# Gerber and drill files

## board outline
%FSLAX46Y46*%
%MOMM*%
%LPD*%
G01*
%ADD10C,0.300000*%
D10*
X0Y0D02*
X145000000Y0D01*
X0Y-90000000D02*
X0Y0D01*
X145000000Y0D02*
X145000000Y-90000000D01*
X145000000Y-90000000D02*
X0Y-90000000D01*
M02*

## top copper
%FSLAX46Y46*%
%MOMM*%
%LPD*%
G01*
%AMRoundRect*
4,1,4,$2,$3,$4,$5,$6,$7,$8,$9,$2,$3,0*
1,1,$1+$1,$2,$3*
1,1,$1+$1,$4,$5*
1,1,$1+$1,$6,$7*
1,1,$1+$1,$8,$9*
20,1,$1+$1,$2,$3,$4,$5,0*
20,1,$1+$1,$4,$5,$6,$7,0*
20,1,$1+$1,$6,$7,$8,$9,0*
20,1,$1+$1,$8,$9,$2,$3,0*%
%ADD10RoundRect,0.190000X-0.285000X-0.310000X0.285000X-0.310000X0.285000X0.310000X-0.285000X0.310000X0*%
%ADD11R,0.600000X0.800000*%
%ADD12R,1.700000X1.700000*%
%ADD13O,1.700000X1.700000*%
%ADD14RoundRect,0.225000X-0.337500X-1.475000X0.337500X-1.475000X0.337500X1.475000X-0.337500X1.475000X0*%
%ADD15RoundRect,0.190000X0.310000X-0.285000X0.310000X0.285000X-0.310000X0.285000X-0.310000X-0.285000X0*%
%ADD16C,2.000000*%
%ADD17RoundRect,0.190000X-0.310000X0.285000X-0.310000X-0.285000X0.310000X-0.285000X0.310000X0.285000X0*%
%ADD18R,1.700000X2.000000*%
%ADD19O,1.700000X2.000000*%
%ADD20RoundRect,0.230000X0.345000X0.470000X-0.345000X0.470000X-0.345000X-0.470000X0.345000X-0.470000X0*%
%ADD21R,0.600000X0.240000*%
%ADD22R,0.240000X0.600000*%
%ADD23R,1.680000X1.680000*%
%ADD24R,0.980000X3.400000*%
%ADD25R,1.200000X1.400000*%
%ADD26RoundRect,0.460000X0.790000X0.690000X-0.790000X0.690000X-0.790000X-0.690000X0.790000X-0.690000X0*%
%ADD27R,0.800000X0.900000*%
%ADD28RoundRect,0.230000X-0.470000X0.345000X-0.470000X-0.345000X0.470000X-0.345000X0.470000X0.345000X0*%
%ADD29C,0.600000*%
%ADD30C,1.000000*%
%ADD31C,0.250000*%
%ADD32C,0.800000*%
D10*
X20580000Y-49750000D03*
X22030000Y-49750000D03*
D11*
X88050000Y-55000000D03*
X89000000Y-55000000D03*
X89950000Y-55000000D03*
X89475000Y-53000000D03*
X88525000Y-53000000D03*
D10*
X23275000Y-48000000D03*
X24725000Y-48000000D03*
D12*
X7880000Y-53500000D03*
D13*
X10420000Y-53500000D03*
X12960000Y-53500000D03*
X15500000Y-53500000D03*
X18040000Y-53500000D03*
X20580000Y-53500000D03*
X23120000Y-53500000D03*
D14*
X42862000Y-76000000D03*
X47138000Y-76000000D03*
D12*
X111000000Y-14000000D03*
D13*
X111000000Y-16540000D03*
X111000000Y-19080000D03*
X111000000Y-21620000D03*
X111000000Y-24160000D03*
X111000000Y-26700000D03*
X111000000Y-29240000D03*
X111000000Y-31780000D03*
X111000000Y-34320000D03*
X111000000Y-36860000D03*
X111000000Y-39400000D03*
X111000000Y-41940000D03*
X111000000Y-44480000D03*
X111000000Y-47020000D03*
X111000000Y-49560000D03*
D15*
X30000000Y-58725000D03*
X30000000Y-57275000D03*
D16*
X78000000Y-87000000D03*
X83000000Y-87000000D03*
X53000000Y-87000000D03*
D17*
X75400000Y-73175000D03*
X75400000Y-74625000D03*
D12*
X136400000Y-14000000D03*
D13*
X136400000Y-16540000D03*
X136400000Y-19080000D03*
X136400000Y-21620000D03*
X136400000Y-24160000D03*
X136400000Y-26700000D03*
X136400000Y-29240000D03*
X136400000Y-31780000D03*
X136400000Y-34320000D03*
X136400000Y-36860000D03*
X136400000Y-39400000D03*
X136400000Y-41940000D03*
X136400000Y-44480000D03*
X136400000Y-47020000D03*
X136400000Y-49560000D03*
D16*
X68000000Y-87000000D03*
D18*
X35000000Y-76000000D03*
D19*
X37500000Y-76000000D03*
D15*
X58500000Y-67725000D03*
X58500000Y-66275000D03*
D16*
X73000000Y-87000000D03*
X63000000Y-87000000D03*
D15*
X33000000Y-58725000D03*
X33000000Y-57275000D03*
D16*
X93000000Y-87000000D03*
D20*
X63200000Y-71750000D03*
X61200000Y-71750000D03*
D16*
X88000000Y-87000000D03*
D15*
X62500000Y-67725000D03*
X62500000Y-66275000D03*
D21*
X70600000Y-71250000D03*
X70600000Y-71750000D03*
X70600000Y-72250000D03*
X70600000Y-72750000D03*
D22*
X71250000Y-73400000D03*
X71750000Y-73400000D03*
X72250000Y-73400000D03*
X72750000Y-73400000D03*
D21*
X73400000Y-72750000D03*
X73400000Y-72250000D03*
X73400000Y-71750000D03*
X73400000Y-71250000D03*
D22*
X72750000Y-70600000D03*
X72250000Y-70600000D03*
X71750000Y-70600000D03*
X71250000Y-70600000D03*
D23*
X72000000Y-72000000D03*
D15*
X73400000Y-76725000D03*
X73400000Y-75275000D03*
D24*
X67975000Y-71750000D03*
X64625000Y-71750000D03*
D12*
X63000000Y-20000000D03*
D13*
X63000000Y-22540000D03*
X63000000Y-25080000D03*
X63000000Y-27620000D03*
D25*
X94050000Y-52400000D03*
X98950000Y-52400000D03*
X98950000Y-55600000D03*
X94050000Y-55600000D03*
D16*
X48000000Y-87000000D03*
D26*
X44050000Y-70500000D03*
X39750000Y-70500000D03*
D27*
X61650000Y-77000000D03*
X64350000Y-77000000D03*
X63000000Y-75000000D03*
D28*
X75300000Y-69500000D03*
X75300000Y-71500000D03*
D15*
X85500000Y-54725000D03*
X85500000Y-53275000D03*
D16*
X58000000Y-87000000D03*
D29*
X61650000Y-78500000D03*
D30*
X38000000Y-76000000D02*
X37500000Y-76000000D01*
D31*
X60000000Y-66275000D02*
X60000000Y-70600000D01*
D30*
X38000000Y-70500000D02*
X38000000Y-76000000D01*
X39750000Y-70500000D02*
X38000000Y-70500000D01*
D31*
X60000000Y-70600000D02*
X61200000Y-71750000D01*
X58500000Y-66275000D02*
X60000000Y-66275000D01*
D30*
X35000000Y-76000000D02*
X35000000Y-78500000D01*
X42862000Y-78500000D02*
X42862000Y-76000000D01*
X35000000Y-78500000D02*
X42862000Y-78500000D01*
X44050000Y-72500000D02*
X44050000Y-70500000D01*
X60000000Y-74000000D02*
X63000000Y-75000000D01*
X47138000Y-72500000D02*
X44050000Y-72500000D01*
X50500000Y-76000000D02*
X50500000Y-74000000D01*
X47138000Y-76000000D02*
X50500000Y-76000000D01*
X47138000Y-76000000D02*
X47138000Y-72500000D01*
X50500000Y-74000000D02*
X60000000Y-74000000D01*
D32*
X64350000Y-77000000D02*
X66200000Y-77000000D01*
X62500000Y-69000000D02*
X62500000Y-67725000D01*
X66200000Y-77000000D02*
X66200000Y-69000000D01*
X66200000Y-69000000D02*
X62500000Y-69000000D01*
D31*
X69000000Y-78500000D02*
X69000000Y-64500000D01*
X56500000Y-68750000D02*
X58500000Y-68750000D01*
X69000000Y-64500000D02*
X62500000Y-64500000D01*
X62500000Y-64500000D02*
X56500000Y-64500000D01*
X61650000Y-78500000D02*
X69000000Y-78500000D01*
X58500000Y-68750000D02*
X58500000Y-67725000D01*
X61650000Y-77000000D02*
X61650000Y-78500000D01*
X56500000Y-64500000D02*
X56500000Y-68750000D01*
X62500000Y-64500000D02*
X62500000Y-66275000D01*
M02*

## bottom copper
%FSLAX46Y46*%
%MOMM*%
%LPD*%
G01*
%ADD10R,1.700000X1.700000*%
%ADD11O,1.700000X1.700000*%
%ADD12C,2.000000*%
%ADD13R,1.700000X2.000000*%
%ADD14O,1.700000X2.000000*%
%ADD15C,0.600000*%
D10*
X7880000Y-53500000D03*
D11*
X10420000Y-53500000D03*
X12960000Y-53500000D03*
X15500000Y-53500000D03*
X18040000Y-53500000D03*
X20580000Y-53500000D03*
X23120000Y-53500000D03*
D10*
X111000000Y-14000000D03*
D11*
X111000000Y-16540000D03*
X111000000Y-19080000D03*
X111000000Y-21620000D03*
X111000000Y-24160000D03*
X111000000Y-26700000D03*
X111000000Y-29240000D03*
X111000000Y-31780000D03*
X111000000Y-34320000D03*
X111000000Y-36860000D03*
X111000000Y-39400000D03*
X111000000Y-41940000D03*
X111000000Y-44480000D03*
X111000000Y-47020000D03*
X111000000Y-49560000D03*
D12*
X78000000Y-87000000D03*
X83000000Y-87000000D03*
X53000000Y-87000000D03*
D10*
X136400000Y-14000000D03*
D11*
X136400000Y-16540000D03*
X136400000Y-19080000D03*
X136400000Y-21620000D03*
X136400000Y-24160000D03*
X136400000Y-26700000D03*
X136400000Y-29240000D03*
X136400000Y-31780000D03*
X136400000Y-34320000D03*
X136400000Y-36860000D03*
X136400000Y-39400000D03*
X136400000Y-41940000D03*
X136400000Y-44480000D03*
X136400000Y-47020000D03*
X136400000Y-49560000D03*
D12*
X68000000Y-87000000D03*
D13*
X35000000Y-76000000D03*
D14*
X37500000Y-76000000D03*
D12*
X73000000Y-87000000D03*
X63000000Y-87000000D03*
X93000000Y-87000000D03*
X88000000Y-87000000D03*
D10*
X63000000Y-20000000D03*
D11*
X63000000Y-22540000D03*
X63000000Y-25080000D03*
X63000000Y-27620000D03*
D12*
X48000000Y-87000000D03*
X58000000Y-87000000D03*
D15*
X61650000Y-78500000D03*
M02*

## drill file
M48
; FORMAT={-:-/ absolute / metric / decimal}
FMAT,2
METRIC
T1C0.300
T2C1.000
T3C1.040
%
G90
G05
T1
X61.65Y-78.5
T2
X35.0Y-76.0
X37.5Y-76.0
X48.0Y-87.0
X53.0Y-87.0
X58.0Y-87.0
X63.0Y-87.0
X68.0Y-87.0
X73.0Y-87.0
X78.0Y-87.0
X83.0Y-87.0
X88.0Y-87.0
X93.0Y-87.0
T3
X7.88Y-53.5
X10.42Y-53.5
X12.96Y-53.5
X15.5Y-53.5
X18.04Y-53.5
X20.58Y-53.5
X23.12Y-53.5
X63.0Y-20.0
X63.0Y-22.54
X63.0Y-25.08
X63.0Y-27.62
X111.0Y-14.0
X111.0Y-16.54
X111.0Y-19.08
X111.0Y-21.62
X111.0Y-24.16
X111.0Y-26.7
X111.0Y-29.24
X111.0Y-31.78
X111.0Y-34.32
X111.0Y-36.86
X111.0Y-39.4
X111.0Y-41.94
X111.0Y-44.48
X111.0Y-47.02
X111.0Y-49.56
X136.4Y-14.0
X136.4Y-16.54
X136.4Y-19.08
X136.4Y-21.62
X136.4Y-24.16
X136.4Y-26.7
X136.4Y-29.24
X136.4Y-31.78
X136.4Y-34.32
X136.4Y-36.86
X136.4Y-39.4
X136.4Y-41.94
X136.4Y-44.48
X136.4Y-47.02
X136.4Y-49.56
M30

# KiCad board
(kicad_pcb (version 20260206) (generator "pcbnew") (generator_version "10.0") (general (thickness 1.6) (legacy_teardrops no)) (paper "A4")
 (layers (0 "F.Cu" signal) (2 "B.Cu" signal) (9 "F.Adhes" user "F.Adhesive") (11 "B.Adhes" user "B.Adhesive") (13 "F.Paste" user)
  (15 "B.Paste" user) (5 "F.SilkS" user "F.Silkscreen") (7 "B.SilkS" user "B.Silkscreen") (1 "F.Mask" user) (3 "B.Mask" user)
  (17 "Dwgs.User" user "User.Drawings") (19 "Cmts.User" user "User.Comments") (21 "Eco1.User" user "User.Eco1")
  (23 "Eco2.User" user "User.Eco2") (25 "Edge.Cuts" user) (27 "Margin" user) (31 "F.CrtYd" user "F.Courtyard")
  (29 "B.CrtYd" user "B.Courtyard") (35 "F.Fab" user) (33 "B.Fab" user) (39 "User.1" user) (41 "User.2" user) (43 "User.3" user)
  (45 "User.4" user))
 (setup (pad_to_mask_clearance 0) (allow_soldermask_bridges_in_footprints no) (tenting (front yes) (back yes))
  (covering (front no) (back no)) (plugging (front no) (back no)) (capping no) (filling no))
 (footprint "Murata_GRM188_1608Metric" (layer "F.Cu") (at 21.305 49.75)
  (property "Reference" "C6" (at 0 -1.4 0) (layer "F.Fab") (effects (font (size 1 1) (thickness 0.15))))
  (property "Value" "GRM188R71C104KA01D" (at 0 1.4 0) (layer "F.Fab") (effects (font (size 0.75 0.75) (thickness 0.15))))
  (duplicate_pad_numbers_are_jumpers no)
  (pad "1" smd roundrect (at -0.725 0) (size 0.95 1) (layers "F.Cu" "F.Mask" "F.Paste") (roundrect_rratio 0.2) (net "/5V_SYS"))
  (pad "2" smd roundrect (at 0.725 0) (size 0.95 1) (layers "F.Cu" "F.Mask" "F.Paste") (roundrect_rratio 0.2) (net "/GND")))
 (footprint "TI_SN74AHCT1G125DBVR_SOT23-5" (layer "F.Cu") (at 89 54)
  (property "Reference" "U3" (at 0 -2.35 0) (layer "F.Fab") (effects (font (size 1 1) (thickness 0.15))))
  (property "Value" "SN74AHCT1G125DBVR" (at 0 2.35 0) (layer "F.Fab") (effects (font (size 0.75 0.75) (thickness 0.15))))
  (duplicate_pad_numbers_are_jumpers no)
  (pad "1" smd rect (at -0.95 1) (size 0.6 0.8) (layers "F.Cu" "F.Mask" "F.Paste") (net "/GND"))
  (pad "2" smd rect (at 0 1) (size 0.6 0.8) (layers "F.Cu" "F.Mask" "F.Paste") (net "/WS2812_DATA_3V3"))
  (pad "3" smd rect (at 0.95 1) (size 0.6 0.8) (layers "F.Cu" "F.Mask" "F.Paste") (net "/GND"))
  (pad "4" smd rect (at 0.475 -1) (size 0.6 0.8) (layers "F.Cu" "F.Mask" "F.Paste") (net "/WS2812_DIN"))
  (pad "5" smd rect (at -0.475 -1) (size 0.6 0.8) (layers "F.Cu" "F.Mask" "F.Paste") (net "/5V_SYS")))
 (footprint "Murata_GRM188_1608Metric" (layer "F.Cu") (at 24 48)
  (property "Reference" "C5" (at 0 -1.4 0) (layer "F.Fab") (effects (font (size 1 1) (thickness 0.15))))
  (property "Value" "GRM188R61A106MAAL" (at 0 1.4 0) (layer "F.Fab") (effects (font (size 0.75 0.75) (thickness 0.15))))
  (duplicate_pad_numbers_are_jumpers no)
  (pad "1" smd roundrect (at -0.725 0) (size 0.95 1) (layers "F.Cu" "F.Mask" "F.Paste") (roundrect_rratio 0.2) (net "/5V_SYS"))
  (pad "2" smd roundrect (at 0.725 0) (size 0.95 1) (layers "F.Cu" "F.Mask" "F.Paste") (roundrect_rratio 0.2) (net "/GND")))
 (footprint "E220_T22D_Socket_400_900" (layer "F.Cu") (at 5 52)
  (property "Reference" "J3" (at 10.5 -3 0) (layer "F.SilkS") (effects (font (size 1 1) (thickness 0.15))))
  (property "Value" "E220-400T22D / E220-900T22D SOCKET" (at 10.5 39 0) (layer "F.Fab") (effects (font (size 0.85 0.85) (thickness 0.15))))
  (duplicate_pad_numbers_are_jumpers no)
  (pad "1" thru_hole rect (at 2.88 1.5) (size 1.7 1.7) (drill 1.04) (layers "*.Cu" "*.Mask") (remove_unused_layers no) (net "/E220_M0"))
  (pad "2" thru_hole oval (at 5.42 1.5) (size 1.7 1.7) (drill 1.04) (layers "*.Cu" "*.Mask") (remove_unused_layers no) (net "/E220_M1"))
  (pad "3" thru_hole oval (at 7.96 1.5) (size 1.7 1.7) (drill 1.04) (layers "*.Cu" "*.Mask") (remove_unused_layers no) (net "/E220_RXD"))
  (pad "4" thru_hole oval (at 10.5 1.5) (size 1.7 1.7) (drill 1.04) (layers "*.Cu" "*.Mask") (remove_unused_layers no) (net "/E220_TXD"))
  (pad "5" thru_hole oval (at 13.04 1.5) (size 1.7 1.7) (drill 1.04) (layers "*.Cu" "*.Mask") (remove_unused_layers no) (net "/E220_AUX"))
  (pad "6" thru_hole oval (at 15.58 1.5) (size 1.7 1.7) (drill 1.04) (layers "*.Cu" "*.Mask") (remove_unused_layers no) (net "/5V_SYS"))
  (pad "7" thru_hole oval (at 18.12 1.5) (size 1.7 1.7) (drill 1.04) (layers "*.Cu" "*.Mask") (remove_unused_layers no) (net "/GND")))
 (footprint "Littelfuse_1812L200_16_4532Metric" (layer "F.Cu") (at 45 76)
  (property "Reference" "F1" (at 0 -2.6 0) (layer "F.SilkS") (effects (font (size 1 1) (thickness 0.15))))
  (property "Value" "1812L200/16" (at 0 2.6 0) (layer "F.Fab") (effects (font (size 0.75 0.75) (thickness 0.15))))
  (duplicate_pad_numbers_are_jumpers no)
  (pad "1" smd roundrect (at -2.138 0) (size 1.125 3.4) (layers "F.Cu" "F.Mask" "F.Paste") (roundrect_rratio 0.2) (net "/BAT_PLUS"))
  (pad "2" smd roundrect (at 2.138 0) (size 1.125 3.4) (layers "F.Cu" "F.Mask" "F.Paste") (roundrect_rratio 0.2) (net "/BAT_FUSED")))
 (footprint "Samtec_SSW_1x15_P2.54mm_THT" (layer "F.Cu") (at 111 14)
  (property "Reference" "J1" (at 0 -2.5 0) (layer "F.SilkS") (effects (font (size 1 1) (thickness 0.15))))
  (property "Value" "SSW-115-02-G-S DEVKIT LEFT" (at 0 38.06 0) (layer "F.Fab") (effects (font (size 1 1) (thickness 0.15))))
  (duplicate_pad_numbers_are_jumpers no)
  (pad "1" thru_hole rect (at 0 0) (size 1.7 1.7) (drill 1.04) (layers "*.Cu" "*.Mask") (remove_unused_layers no) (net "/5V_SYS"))
  (pad "2" thru_hole oval (at 0 2.54) (size 1.7 1.7) (drill 1.04) (layers "*.Cu" "*.Mask") (remove_unused_layers no) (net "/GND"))
  (pad "3" thru_hole oval (at 0 5.08) (size 1.7 1.7) (drill 1.04) (layers "*.Cu" "*.Mask") (remove_unused_layers no))
  (pad "4" thru_hole oval (at 0 7.62) (size 1.7 1.7) (drill 1.04) (layers "*.Cu" "*.Mask") (remove_unused_layers no))
  (pad "5" thru_hole oval (at 0 10.16) (size 1.7 1.7) (drill 1.04) (layers "*.Cu" "*.Mask") (remove_unused_layers no))
  (pad "6" thru_hole oval (at 0 12.7) (size 1.7 1.7) (drill 1.04) (layers "*.Cu" "*.Mask") (remove_unused_layers no) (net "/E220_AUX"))
  (pad "7" thru_hole oval (at 0 15.24) (size 1.7 1.7) (drill 1.04) (layers "*.Cu" "*.Mask") (remove_unused_layers no) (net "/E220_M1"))
  (pad "8" thru_hole oval (at 0 17.78) (size 1.7 1.7) (drill 1.04) (layers "*.Cu" "*.Mask") (remove_unused_layers no) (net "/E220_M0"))
  (pad "9" thru_hole oval (at 0 20.32) (size 1.7 1.7) (drill 1.04) (layers "*.Cu" "*.Mask") (remove_unused_layers no))
  (pad "10" thru_hole oval (at 0 22.86) (size 1.7 1.7) (drill 1.04) (layers "*.Cu" "*.Mask") (remove_unused_layers no))
  (pad "11" thru_hole oval (at 0 25.4) (size 1.7 1.7) (drill 1.04) (layers "*.Cu" "*.Mask") (remove_unused_layers no))
  (pad "12" thru_hole oval (at 0 27.94) (size 1.7 1.7) (drill 1.04) (layers "*.Cu" "*.Mask") (remove_unused_layers no))
  (pad "13" thru_hole oval (at 0 30.48) (size 1.7 1.7) (drill 1.04) (layers "*.Cu" "*.Mask") (remove_unused_layers no))
  (pad "14" thru_hole oval (at 0 33.02) (size 1.7 1.7) (drill 1.04) (layers "*.Cu" "*.Mask") (remove_unused_layers no))
  (pad "15" thru_hole oval (at 0 35.56) (size 1.7 1.7) (drill 1.04) (layers "*.Cu" "*.Mask") (remove_unused_layers no)))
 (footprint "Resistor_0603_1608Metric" (layer "F.Cu") (at 30 58 90)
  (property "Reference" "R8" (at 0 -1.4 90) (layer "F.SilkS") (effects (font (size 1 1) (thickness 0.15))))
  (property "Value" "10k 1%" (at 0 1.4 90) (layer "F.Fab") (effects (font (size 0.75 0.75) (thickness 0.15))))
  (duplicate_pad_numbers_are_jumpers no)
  (pad "1" smd roundrect (at -0.725 0 90) (size 0.95 1) (layers "F.Cu" "F.Mask" "F.Paste") (roundrect_rratio 0.2) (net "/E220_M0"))
  (pad "2" smd roundrect (at 0.725 0 90) (size 0.95 1) (layers "F.Cu" "F.Mask" "F.Paste") (roundrect_rratio 0.2) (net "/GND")))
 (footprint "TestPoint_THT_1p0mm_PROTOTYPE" (layer "F.Cu") (at 78 87)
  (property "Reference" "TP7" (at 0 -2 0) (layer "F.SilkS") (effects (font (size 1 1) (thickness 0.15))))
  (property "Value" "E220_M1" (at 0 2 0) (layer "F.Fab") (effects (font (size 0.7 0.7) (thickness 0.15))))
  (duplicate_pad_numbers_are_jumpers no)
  (pad "1" thru_hole circle (at 0 0) (size 2 2) (drill 1) (layers "*.Cu" "*.Mask") (remove_unused_layers no) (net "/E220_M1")))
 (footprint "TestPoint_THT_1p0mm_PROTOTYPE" (layer "F.Cu") (at 83 87)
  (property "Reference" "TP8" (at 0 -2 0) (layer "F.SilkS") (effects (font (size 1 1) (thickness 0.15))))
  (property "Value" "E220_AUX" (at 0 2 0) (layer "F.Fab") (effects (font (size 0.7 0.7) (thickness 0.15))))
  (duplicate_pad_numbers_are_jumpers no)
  (pad "1" thru_hole circle (at 0 0) (size 2 2) (drill 1) (layers "*.Cu" "*.Mask") (remove_unused_layers no) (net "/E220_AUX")))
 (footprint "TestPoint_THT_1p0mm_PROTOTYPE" (layer "F.Cu") (at 53 87)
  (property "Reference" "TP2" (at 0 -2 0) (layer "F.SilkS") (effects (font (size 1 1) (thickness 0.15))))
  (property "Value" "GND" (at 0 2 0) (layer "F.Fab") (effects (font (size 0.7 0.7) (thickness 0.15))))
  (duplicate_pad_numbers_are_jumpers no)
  (pad "1" thru_hole circle (at 0 0) (size 2 2) (drill 1) (layers "*.Cu" "*.Mask") (remove_unused_layers no) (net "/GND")))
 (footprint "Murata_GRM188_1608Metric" (layer "F.Cu") (at 75.4 73.9 -90)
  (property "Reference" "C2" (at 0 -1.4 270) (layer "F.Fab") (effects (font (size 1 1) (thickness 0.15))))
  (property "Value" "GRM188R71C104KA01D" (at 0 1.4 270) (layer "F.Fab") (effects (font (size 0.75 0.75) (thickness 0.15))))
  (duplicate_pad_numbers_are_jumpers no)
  (pad "1" smd roundrect (at -0.725 0 270) (size 0.95 1) (layers "F.Cu" "F.Mask" "F.Paste") (roundrect_rratio 0.2) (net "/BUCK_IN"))
  (pad "2" smd roundrect (at 0.725 0 270) (size 0.95 1) (layers "F.Cu" "F.Mask" "F.Paste") (roundrect_rratio 0.2) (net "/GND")))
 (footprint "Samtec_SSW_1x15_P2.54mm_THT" (layer "F.Cu") (at 136.4 14)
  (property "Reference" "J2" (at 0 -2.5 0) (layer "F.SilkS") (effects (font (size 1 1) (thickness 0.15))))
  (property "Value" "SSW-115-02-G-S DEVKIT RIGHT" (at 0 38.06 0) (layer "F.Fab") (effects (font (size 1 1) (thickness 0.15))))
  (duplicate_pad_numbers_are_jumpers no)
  (pad "1" thru_hole rect (at 0 0) (size 1.7 1.7) (drill 1.04) (layers "*.Cu" "*.Mask") (remove_unused_layers no) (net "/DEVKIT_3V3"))
  (pad "2" thru_hole oval (at 0 2.54) (size 1.7 1.7) (drill 1.04) (layers "*.Cu" "*.Mask") (remove_unused_layers no) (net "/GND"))
  (pad "3" thru_hole oval (at 0 5.08) (size 1.7 1.7) (drill 1.04) (layers "*.Cu" "*.Mask") (remove_unused_layers no))
  (pad "4" thru_hole oval (at 0 7.62) (size 1.7 1.7) (drill 1.04) (layers "*.Cu" "*.Mask") (remove_unused_layers no))
  (pad "5" thru_hole oval (at 0 10.16) (size 1.7 1.7) (drill 1.04) (layers "*.Cu" "*.Mask") (remove_unused_layers no)
   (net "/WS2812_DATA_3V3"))
  (pad "6" thru_hole oval (at 0 12.7) (size 1.7 1.7) (drill 1.04) (layers "*.Cu" "*.Mask") (remove_unused_layers no) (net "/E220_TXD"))
  (pad "7" thru_hole oval (at 0 15.24) (size 1.7 1.7) (drill 1.04) (layers "*.Cu" "*.Mask") (remove_unused_layers no) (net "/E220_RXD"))
  (pad "8" thru_hole oval (at 0 17.78) (size 1.7 1.7) (drill 1.04) (layers "*.Cu" "*.Mask") (remove_unused_layers no))
  (pad "9" thru_hole oval (at 0 20.32) (size 1.7 1.7) (drill 1.04) (layers "*.Cu" "*.Mask") (remove_unused_layers no))
  (pad "10" thru_hole oval (at 0 22.86) (size 1.7 1.7) (drill 1.04) (layers "*.Cu" "*.Mask") (remove_unused_layers no))
  (pad "11" thru_hole oval (at 0 25.4) (size 1.7 1.7) (drill 1.04) (layers "*.Cu" "*.Mask") (remove_unused_layers no) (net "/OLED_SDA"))
  (pad "12" thru_hole oval (at 0 27.94) (size 1.7 1.7) (drill 1.04) (layers "*.Cu" "*.Mask") (remove_unused_layers no))
  (pad "13" thru_hole oval (at 0 30.48) (size 1.7 1.7) (drill 1.04) (layers "*.Cu" "*.Mask") (remove_unused_layers no))
  (pad "14" thru_hole oval (at 0 33.02) (size 1.7 1.7) (drill 1.04) (layers "*.Cu" "*.Mask") (remove_unused_layers no) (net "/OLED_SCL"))
  (pad "15" thru_hole oval (at 0 35.56) (size 1.7 1.7) (drill 1.04) (layers "*.Cu" "*.Mask") (remove_unused_layers no)))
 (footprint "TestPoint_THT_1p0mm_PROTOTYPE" (layer "F.Cu") (at 68 87)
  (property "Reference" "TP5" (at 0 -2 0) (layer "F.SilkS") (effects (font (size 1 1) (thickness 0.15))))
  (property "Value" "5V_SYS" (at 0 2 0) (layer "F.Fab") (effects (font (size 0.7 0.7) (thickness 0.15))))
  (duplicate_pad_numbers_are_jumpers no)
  (pad "1" thru_hole circle (at 0 0) (size 2 2) (drill 1) (layers "*.Cu" "*.Mask") (remove_unused_layers no) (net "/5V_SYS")))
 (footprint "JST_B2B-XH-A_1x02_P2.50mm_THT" (layer "F.Cu") (at 35 76)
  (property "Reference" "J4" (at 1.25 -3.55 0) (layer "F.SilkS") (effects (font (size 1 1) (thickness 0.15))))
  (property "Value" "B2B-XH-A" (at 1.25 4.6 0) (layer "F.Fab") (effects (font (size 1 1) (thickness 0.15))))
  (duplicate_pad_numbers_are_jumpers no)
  (pad "1" thru_hole rect (at 0 0) (size 1.7 2) (drill 1) (layers "*.Cu" "*.Mask") (remove_unused_layers no) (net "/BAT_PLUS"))
  (pad "2" thru_hole oval (at 2.5 0) (size 1.7 2) (drill 1) (layers "*.Cu" "*.Mask") (remove_unused_layers no) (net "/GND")))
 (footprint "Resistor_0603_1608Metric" (layer "F.Cu") (at 58.5 67 90)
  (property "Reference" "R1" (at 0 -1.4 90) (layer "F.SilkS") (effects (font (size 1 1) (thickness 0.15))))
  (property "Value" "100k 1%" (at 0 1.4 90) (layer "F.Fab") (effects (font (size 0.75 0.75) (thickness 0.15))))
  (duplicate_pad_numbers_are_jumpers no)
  (pad "1" smd roundrect (at -0.725 0 90) (size 0.95 1) (layers "F.Cu" "F.Mask" "F.Paste") (roundrect_rratio 0.2) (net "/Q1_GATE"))
  (pad "2" smd roundrect (at 0.725 0 90) (size 0.95 1) (layers "F.Cu" "F.Mask" "F.Paste") (roundrect_rratio 0.2) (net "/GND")))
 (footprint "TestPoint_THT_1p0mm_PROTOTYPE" (layer "F.Cu") (at 73 87)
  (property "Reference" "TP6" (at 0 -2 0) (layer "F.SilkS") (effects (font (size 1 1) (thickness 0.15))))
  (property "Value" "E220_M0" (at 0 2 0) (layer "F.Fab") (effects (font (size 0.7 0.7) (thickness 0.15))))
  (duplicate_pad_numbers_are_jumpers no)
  (pad "1" thru_hole circle (at 0 0) (size 2 2) (drill 1) (layers "*.Cu" "*.Mask") (remove_unused_layers no) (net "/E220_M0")))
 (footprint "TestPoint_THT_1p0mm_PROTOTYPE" (layer "F.Cu") (at 63 87)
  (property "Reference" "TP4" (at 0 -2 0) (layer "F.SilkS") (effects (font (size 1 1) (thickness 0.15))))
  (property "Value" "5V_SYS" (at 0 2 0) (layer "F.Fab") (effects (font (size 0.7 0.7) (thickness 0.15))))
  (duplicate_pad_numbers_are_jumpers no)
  (pad "1" thru_hole circle (at 0 0) (size 2 2) (drill 1) (layers "*.Cu" "*.Mask") (remove_unused_layers no) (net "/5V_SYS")))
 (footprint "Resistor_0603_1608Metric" (layer "F.Cu") (at 33 58 90)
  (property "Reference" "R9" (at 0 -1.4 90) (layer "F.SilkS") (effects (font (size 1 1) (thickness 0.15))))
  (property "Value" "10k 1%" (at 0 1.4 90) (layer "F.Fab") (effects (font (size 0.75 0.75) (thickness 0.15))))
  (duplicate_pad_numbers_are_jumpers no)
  (pad "1" smd roundrect (at -0.725 0 90) (size 0.95 1) (layers "F.Cu" "F.Mask" "F.Paste") (roundrect_rratio 0.2) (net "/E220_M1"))
  (pad "2" smd roundrect (at 0.725 0 90) (size 0.95 1) (layers "F.Cu" "F.Mask" "F.Paste") (roundrect_rratio 0.2) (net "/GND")))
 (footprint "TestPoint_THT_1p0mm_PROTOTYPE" (layer "F.Cu") (at 93 87)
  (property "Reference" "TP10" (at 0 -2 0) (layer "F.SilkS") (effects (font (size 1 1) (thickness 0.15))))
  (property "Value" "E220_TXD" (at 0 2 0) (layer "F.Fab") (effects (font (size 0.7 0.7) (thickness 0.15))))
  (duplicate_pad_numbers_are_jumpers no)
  (pad "1" thru_hole circle (at 0 0) (size 2 2) (drill 1) (layers "*.Cu" "*.Mask") (remove_unused_layers no) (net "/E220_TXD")))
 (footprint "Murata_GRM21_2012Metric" (layer "F.Cu") (at 62.2 71.75 180)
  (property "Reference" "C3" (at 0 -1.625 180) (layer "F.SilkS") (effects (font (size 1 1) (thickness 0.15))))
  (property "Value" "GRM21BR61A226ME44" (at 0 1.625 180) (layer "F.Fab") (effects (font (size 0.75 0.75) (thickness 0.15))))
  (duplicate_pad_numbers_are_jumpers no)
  (pad "1" smd roundrect (at -1 0 180) (size 1.15 1.4) (layers "F.Cu" "F.Mask" "F.Paste") (roundrect_rratio 0.2) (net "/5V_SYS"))
  (pad "2" smd roundrect (at 1 0 180) (size 1.15 1.4) (layers "F.Cu" "F.Mask" "F.Paste") (roundrect_rratio 0.2) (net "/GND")))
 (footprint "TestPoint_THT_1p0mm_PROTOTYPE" (layer "F.Cu") (at 88 87)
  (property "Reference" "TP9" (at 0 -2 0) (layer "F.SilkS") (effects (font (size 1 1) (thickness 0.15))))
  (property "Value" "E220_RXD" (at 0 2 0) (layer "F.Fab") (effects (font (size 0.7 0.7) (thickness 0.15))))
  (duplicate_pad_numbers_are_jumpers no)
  (pad "1" thru_hole circle (at 0 0) (size 2 2) (drill 1) (layers "*.Cu" "*.Mask") (remove_unused_layers no) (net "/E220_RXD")))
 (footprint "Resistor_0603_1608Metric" (layer "F.Cu") (at 62.5 67 90)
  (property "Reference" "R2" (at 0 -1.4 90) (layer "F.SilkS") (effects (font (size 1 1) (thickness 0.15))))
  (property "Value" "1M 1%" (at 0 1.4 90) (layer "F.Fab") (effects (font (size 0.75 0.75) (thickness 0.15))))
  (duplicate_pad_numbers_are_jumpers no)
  (pad "1" smd roundrect (at -0.725 0 90) (size 0.95 1) (layers "F.Cu" "F.Mask" "F.Paste") (roundrect_rratio 0.2) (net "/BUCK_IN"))
  (pad "2" smd roundrect (at 0.725 0 90) (size 0.95 1) (layers "F.Cu" "F.Mask" "F.Paste") (roundrect_rratio 0.2) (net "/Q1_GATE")))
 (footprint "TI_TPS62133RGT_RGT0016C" (layer "F.Cu") (at 72 72)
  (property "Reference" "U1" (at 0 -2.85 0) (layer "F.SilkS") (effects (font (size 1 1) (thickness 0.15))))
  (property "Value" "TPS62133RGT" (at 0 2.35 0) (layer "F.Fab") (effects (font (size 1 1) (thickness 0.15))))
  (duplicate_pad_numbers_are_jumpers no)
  (pad "" smd rect (at 0 0) (size 1.55 1.55) (layers "F.Paste"))
  (pad "1" smd rect (at -1.4 -0.75) (size 0.6 0.24) (layers "F.Cu" "F.Mask" "F.Paste") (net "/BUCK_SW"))
  (pad "2" smd rect (at -1.4 -0.25) (size 0.6 0.24) (layers "F.Cu" "F.Mask" "F.Paste") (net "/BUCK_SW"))
  (pad "3" smd rect (at -1.4 0.25) (size 0.6 0.24) (layers "F.Cu" "F.Mask" "F.Paste") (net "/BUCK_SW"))
  (pad "4" smd rect (at -1.4 0.75) (size 0.6 0.24) (layers "F.Cu" "F.Mask" "F.Paste"))
  (pad "5" smd rect (at -0.75 1.4) (size 0.24 0.6) (layers "F.Cu" "F.Mask" "F.Paste") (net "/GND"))
  (pad "6" smd rect (at -0.25 1.4) (size 0.24 0.6) (layers "F.Cu" "F.Mask" "F.Paste") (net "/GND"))
  (pad "7" smd rect (at 0.25 1.4) (size 0.24 0.6) (layers "F.Cu" "F.Mask" "F.Paste") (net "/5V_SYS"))
  (pad "8" smd rect (at 0.75 1.4) (size 0.24 0.6) (layers "F.Cu" "F.Mask" "F.Paste") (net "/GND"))
  (pad "9" smd rect (at 1.4 0.75) (size 0.6 0.24) (layers "F.Cu" "F.Mask" "F.Paste") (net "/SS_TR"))
  (pad "10" smd rect (at 1.4 0.25) (size 0.6 0.24) (layers "F.Cu" "F.Mask" "F.Paste") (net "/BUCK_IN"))
  (pad "11" smd rect (at 1.4 -0.25) (size 0.6 0.24) (layers "F.Cu" "F.Mask" "F.Paste") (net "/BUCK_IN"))
  (pad "12" smd rect (at 1.4 -0.75) (size 0.6 0.24) (layers "F.Cu" "F.Mask" "F.Paste") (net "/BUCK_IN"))
  (pad "13" smd rect (at 0.75 -1.4) (size 0.24 0.6) (layers "F.Cu" "F.Mask" "F.Paste") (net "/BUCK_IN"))
  (pad "14" smd rect (at 0.25 -1.4) (size 0.24 0.6) (layers "F.Cu" "F.Mask" "F.Paste") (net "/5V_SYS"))
  (pad "15" smd rect (at -0.25 -1.4) (size 0.24 0.6) (layers "F.Cu" "F.Mask" "F.Paste") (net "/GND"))
  (pad "16" smd rect (at -0.75 -1.4) (size 0.24 0.6) (layers "F.Cu" "F.Mask" "F.Paste") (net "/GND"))
  (pad "EP" smd rect (at 0 0) (size 1.68 1.68) (layers "F.Cu" "F.Mask") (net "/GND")))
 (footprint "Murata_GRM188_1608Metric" (layer "F.Cu") (at 73.4 76 90)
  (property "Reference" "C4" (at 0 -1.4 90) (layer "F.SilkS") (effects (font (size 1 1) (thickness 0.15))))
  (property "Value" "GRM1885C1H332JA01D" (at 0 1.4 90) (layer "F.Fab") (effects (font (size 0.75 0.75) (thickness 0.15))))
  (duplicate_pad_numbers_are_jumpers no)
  (pad "1" smd roundrect (at -0.725 0 90) (size 0.95 1) (layers "F.Cu" "F.Mask" "F.Paste") (roundrect_rratio 0.2) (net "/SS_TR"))
  (pad "2" smd roundrect (at 0.725 0 90) (size 0.95 1) (layers "F.Cu" "F.Mask" "F.Paste") (roundrect_rratio 0.2) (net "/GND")))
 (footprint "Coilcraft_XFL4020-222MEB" (layer "F.Cu") (at 66.3 71.75 180)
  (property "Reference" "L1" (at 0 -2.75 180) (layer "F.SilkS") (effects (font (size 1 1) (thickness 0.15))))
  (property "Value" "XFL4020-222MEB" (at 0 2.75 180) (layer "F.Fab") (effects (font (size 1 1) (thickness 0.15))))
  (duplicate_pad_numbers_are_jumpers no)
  (pad "1" smd rect (at -1.675 0 180) (size 0.98 3.4) (layers "F.Cu" "F.Mask" "F.Paste") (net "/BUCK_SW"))
  (pad "2" smd rect (at 1.675 0 180) (size 0.98 3.4) (layers "F.Cu" "F.Mask" "F.Paste") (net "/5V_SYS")))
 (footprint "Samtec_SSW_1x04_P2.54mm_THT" (layer "F.Cu") (at 63 20)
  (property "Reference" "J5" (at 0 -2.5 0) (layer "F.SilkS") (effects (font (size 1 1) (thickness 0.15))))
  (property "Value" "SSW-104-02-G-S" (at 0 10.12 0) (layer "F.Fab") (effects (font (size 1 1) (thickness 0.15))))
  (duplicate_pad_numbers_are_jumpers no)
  (pad "1" thru_hole rect (at 0 0) (size 1.7 1.7) (drill 1.04) (layers "*.Cu" "*.Mask") (remove_unused_layers no) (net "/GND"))
  (pad "2" thru_hole oval (at 0 2.54) (size 1.7 1.7) (drill 1.04) (layers "*.Cu" "*.Mask") (remove_unused_layers no) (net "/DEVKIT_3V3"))
  (pad "3" thru_hole oval (at 0 5.08) (size 1.7 1.7) (drill 1.04) (layers "*.Cu" "*.Mask") (remove_unused_layers no) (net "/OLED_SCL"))
  (pad "4" thru_hole oval (at 0 7.62) (size 1.7 1.7) (drill 1.04) (layers "*.Cu" "*.Mask") (remove_unused_layers no) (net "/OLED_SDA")))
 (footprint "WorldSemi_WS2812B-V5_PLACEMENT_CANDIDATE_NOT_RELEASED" (layer "F.Cu") (at 96.5 54)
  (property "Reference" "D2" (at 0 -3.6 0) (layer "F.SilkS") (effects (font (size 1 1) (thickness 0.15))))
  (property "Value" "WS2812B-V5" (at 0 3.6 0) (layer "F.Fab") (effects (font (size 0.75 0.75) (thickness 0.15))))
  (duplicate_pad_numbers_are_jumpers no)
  (pad "1" smd rect (at -2.45 -1.6) (size 1.2 1.4) (layers "F.Cu" "F.Mask" "F.Paste") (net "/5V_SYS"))
  (pad "2" smd rect (at 2.45 -1.6) (size 1.2 1.4) (layers "F.Cu" "F.Mask" "F.Paste"))
  (pad "3" smd rect (at 2.45 1.6) (size 1.2 1.4) (layers "F.Cu" "F.Mask" "F.Paste") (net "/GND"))
  (pad "4" smd rect (at -2.45 1.6) (size 1.2 1.4) (layers "F.Cu" "F.Mask" "F.Paste") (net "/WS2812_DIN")))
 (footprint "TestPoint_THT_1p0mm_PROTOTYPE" (layer "F.Cu") (at 48 87)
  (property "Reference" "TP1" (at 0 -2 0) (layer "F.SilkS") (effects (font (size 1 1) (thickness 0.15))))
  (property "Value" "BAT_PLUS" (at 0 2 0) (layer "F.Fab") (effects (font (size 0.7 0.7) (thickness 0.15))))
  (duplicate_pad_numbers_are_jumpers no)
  (pad "1" thru_hole circle (at 0 0) (size 2 2) (drill 1) (layers "*.Cu" "*.Mask") (remove_unused_layers no) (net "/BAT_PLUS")))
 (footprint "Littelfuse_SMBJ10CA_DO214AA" (layer "F.Cu") (at 41.9 70.5 180)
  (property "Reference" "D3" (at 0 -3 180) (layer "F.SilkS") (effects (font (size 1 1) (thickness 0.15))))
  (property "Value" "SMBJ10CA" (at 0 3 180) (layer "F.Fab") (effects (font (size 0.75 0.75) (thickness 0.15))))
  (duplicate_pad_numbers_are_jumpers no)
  (pad "1" smd roundrect (at -2.15 0 180) (size 2.5 2.3) (layers "F.Cu" "F.Mask" "F.Paste") (roundrect_rratio 0.2) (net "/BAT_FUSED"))
  (pad "2" smd roundrect (at 2.15 0 180) (size 2.5 2.3) (layers "F.Cu" "F.Mask" "F.Paste") (roundrect_rratio 0.2) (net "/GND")))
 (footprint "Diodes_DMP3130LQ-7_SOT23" (layer "F.Cu") (at 63 76)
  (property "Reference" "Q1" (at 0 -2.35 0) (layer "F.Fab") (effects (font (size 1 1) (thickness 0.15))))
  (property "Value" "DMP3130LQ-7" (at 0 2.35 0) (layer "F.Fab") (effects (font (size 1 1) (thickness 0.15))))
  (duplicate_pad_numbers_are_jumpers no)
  (pad "1" smd rect (at -1.35 1) (size 0.8 0.9) (layers "F.Cu" "F.Mask" "F.Paste") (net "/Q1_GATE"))
  (pad "2" smd rect (at 1.35 1) (size 0.8 0.9) (layers "F.Cu" "F.Mask" "F.Paste") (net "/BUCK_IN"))
  (pad "3" smd rect (at 0 -1) (size 0.8 0.9) (layers "F.Cu" "F.Mask" "F.Paste") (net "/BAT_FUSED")))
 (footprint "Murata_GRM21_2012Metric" (layer "F.Cu") (at 75.3 70.5 -90)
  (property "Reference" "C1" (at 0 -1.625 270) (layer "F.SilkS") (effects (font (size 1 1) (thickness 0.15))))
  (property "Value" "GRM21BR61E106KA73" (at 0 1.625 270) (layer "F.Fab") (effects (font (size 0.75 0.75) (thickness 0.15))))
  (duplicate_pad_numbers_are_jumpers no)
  (pad "1" smd roundrect (at -1 0 270) (size 1.15 1.4) (layers "F.Cu" "F.Mask" "F.Paste") (roundrect_rratio 0.2) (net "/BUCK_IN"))
  (pad "2" smd roundrect (at 1 0 270) (size 1.15 1.4) (layers "F.Cu" "F.Mask" "F.Paste") (roundrect_rratio 0.2) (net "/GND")))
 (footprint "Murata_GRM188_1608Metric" (layer "F.Cu") (at 85.5 54 90)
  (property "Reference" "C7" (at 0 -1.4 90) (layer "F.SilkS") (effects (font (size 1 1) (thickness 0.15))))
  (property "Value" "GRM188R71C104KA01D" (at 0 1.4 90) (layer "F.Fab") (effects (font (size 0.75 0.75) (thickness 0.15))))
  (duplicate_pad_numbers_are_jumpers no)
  (pad "1" smd roundrect (at -0.725 0 90) (size 0.95 1) (layers "F.Cu" "F.Mask" "F.Paste") (roundrect_rratio 0.2) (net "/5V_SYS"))
  (pad "2" smd roundrect (at 0.725 0 90) (size 0.95 1) (layers "F.Cu" "F.Mask" "F.Paste") (roundrect_rratio 0.2) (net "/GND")))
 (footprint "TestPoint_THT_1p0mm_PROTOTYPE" (layer "F.Cu") (at 58 87)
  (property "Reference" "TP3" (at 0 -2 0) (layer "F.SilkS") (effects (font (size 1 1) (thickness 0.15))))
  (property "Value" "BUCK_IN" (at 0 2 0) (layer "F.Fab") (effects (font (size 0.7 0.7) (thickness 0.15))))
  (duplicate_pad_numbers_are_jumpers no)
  (pad "1" thru_hole circle (at 0 0) (size 2 2) (drill 1) (layers "*.Cu" "*.Mask") (remove_unused_layers no) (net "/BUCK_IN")))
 (gr_line (start 0 0) (end 145 0) (stroke (width 0.3) (type default)) (layer "Edge.Cuts"))
 (gr_line (start 0 90) (end 0 0) (stroke (width 0.3) (type default)) (layer "Edge.Cuts"))
 (gr_line (start 145 0) (end 145 90) (stroke (width 0.3) (type default)) (layer "Edge.Cuts"))
 (gr_line (start 145 90) (end 0 90) (stroke (width 0.3) (type default)) (layer "Edge.Cuts"))
 (segment (start 38 76) (end 37.5 76) (width 1) (layer "F.Cu") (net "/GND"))
 (segment (start 60 66.275) (end 60 70.6) (width 0.25) (layer "F.Cu") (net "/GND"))
 (segment (start 38 70.5) (end 38 76) (width 1) (layer "F.Cu") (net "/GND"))
 (segment (start 39.75 70.5) (end 38 70.5) (width 1) (layer "F.Cu") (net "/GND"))
 (segment (start 60 70.6) (end 61.2 71.75) (width 0.25) (layer "F.Cu") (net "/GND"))
 (segment (start 58.5 66.275) (end 60 66.275) (width 0.25) (layer "F.Cu") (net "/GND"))
 (segment (start 35 76) (end 35 78.5) (width 1) (layer "F.Cu") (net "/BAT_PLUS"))
 (segment (start 42.862 78.5) (end 42.862 76) (width 1) (layer "F.Cu") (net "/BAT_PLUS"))
 (segment (start 35 78.5) (end 42.862 78.5) (width 1) (layer "F.Cu") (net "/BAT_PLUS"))
 (segment (start 44.05 72.5) (end 44.05 70.5) (width 1) (layer "F.Cu") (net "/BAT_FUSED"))
 (segment (start 60 74) (end 63 75) (width 1) (layer "F.Cu") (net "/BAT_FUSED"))
 (segment (start 47.138 72.5) (end 44.05 72.5) (width 1) (layer "F.Cu") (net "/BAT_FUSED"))
 (segment (start 50.5 76) (end 50.5 74) (width 1) (layer "F.Cu") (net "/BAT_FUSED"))
 (segment (start 47.138 76) (end 50.5 76) (width 1) (layer "F.Cu") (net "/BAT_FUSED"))
 (segment (start 47.138 76) (end 47.138 72.5) (width 1) (layer "F.Cu") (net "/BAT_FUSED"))
 (segment (start 50.5 74) (end 60 74) (width 1) (layer "F.Cu") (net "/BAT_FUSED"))
 (segment (start 64.35 77) (end 66.2 77) (width 0.8) (layer "F.Cu") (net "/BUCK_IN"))
 (segment (start 62.5 69) (end 62.5 67.725) (width 0.8) (layer "F.Cu") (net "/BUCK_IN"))
 (segment (start 66.2 77) (end 66.2 69) (width 0.8) (layer "F.Cu") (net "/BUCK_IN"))
 (segment (start 66.2 69) (end 62.5 69) (width 0.8) (layer "F.Cu") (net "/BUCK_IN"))
 (segment (start 69 78.5) (end 69 64.5) (width 0.25) (layer "F.Cu") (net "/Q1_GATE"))
 (segment (start 56.5 68.75) (end 58.5 68.75) (width 0.25) (layer "F.Cu") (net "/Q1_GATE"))
 (segment (start 69 64.5) (end 62.5 64.5) (width 0.25) (layer "F.Cu") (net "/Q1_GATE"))
 (segment (start 62.5 64.5) (end 56.5 64.5) (width 0.25) (layer "F.Cu") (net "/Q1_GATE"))
 (segment (start 61.65 78.5) (end 69 78.5) (width 0.25) (layer "F.Cu") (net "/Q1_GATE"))
 (segment (start 58.5 68.75) (end 58.5 67.725) (width 0.25) (layer "F.Cu") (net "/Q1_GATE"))
 (segment (start 61.65 77) (end 61.65 78.5) (width 0.25) (layer "F.Cu") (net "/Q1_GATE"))
 (segment (start 56.5 64.5) (end 56.5 68.75) (width 0.25) (layer "F.Cu") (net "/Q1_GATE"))
 (segment (start 62.5 64.5) (end 62.5 66.275) (width 0.25) (layer "F.Cu") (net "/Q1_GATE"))
 (via (at 61.65 78.5) (size 0.6) (drill 0.3) (layers "F.Cu" "B.Cu") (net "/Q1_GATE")))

